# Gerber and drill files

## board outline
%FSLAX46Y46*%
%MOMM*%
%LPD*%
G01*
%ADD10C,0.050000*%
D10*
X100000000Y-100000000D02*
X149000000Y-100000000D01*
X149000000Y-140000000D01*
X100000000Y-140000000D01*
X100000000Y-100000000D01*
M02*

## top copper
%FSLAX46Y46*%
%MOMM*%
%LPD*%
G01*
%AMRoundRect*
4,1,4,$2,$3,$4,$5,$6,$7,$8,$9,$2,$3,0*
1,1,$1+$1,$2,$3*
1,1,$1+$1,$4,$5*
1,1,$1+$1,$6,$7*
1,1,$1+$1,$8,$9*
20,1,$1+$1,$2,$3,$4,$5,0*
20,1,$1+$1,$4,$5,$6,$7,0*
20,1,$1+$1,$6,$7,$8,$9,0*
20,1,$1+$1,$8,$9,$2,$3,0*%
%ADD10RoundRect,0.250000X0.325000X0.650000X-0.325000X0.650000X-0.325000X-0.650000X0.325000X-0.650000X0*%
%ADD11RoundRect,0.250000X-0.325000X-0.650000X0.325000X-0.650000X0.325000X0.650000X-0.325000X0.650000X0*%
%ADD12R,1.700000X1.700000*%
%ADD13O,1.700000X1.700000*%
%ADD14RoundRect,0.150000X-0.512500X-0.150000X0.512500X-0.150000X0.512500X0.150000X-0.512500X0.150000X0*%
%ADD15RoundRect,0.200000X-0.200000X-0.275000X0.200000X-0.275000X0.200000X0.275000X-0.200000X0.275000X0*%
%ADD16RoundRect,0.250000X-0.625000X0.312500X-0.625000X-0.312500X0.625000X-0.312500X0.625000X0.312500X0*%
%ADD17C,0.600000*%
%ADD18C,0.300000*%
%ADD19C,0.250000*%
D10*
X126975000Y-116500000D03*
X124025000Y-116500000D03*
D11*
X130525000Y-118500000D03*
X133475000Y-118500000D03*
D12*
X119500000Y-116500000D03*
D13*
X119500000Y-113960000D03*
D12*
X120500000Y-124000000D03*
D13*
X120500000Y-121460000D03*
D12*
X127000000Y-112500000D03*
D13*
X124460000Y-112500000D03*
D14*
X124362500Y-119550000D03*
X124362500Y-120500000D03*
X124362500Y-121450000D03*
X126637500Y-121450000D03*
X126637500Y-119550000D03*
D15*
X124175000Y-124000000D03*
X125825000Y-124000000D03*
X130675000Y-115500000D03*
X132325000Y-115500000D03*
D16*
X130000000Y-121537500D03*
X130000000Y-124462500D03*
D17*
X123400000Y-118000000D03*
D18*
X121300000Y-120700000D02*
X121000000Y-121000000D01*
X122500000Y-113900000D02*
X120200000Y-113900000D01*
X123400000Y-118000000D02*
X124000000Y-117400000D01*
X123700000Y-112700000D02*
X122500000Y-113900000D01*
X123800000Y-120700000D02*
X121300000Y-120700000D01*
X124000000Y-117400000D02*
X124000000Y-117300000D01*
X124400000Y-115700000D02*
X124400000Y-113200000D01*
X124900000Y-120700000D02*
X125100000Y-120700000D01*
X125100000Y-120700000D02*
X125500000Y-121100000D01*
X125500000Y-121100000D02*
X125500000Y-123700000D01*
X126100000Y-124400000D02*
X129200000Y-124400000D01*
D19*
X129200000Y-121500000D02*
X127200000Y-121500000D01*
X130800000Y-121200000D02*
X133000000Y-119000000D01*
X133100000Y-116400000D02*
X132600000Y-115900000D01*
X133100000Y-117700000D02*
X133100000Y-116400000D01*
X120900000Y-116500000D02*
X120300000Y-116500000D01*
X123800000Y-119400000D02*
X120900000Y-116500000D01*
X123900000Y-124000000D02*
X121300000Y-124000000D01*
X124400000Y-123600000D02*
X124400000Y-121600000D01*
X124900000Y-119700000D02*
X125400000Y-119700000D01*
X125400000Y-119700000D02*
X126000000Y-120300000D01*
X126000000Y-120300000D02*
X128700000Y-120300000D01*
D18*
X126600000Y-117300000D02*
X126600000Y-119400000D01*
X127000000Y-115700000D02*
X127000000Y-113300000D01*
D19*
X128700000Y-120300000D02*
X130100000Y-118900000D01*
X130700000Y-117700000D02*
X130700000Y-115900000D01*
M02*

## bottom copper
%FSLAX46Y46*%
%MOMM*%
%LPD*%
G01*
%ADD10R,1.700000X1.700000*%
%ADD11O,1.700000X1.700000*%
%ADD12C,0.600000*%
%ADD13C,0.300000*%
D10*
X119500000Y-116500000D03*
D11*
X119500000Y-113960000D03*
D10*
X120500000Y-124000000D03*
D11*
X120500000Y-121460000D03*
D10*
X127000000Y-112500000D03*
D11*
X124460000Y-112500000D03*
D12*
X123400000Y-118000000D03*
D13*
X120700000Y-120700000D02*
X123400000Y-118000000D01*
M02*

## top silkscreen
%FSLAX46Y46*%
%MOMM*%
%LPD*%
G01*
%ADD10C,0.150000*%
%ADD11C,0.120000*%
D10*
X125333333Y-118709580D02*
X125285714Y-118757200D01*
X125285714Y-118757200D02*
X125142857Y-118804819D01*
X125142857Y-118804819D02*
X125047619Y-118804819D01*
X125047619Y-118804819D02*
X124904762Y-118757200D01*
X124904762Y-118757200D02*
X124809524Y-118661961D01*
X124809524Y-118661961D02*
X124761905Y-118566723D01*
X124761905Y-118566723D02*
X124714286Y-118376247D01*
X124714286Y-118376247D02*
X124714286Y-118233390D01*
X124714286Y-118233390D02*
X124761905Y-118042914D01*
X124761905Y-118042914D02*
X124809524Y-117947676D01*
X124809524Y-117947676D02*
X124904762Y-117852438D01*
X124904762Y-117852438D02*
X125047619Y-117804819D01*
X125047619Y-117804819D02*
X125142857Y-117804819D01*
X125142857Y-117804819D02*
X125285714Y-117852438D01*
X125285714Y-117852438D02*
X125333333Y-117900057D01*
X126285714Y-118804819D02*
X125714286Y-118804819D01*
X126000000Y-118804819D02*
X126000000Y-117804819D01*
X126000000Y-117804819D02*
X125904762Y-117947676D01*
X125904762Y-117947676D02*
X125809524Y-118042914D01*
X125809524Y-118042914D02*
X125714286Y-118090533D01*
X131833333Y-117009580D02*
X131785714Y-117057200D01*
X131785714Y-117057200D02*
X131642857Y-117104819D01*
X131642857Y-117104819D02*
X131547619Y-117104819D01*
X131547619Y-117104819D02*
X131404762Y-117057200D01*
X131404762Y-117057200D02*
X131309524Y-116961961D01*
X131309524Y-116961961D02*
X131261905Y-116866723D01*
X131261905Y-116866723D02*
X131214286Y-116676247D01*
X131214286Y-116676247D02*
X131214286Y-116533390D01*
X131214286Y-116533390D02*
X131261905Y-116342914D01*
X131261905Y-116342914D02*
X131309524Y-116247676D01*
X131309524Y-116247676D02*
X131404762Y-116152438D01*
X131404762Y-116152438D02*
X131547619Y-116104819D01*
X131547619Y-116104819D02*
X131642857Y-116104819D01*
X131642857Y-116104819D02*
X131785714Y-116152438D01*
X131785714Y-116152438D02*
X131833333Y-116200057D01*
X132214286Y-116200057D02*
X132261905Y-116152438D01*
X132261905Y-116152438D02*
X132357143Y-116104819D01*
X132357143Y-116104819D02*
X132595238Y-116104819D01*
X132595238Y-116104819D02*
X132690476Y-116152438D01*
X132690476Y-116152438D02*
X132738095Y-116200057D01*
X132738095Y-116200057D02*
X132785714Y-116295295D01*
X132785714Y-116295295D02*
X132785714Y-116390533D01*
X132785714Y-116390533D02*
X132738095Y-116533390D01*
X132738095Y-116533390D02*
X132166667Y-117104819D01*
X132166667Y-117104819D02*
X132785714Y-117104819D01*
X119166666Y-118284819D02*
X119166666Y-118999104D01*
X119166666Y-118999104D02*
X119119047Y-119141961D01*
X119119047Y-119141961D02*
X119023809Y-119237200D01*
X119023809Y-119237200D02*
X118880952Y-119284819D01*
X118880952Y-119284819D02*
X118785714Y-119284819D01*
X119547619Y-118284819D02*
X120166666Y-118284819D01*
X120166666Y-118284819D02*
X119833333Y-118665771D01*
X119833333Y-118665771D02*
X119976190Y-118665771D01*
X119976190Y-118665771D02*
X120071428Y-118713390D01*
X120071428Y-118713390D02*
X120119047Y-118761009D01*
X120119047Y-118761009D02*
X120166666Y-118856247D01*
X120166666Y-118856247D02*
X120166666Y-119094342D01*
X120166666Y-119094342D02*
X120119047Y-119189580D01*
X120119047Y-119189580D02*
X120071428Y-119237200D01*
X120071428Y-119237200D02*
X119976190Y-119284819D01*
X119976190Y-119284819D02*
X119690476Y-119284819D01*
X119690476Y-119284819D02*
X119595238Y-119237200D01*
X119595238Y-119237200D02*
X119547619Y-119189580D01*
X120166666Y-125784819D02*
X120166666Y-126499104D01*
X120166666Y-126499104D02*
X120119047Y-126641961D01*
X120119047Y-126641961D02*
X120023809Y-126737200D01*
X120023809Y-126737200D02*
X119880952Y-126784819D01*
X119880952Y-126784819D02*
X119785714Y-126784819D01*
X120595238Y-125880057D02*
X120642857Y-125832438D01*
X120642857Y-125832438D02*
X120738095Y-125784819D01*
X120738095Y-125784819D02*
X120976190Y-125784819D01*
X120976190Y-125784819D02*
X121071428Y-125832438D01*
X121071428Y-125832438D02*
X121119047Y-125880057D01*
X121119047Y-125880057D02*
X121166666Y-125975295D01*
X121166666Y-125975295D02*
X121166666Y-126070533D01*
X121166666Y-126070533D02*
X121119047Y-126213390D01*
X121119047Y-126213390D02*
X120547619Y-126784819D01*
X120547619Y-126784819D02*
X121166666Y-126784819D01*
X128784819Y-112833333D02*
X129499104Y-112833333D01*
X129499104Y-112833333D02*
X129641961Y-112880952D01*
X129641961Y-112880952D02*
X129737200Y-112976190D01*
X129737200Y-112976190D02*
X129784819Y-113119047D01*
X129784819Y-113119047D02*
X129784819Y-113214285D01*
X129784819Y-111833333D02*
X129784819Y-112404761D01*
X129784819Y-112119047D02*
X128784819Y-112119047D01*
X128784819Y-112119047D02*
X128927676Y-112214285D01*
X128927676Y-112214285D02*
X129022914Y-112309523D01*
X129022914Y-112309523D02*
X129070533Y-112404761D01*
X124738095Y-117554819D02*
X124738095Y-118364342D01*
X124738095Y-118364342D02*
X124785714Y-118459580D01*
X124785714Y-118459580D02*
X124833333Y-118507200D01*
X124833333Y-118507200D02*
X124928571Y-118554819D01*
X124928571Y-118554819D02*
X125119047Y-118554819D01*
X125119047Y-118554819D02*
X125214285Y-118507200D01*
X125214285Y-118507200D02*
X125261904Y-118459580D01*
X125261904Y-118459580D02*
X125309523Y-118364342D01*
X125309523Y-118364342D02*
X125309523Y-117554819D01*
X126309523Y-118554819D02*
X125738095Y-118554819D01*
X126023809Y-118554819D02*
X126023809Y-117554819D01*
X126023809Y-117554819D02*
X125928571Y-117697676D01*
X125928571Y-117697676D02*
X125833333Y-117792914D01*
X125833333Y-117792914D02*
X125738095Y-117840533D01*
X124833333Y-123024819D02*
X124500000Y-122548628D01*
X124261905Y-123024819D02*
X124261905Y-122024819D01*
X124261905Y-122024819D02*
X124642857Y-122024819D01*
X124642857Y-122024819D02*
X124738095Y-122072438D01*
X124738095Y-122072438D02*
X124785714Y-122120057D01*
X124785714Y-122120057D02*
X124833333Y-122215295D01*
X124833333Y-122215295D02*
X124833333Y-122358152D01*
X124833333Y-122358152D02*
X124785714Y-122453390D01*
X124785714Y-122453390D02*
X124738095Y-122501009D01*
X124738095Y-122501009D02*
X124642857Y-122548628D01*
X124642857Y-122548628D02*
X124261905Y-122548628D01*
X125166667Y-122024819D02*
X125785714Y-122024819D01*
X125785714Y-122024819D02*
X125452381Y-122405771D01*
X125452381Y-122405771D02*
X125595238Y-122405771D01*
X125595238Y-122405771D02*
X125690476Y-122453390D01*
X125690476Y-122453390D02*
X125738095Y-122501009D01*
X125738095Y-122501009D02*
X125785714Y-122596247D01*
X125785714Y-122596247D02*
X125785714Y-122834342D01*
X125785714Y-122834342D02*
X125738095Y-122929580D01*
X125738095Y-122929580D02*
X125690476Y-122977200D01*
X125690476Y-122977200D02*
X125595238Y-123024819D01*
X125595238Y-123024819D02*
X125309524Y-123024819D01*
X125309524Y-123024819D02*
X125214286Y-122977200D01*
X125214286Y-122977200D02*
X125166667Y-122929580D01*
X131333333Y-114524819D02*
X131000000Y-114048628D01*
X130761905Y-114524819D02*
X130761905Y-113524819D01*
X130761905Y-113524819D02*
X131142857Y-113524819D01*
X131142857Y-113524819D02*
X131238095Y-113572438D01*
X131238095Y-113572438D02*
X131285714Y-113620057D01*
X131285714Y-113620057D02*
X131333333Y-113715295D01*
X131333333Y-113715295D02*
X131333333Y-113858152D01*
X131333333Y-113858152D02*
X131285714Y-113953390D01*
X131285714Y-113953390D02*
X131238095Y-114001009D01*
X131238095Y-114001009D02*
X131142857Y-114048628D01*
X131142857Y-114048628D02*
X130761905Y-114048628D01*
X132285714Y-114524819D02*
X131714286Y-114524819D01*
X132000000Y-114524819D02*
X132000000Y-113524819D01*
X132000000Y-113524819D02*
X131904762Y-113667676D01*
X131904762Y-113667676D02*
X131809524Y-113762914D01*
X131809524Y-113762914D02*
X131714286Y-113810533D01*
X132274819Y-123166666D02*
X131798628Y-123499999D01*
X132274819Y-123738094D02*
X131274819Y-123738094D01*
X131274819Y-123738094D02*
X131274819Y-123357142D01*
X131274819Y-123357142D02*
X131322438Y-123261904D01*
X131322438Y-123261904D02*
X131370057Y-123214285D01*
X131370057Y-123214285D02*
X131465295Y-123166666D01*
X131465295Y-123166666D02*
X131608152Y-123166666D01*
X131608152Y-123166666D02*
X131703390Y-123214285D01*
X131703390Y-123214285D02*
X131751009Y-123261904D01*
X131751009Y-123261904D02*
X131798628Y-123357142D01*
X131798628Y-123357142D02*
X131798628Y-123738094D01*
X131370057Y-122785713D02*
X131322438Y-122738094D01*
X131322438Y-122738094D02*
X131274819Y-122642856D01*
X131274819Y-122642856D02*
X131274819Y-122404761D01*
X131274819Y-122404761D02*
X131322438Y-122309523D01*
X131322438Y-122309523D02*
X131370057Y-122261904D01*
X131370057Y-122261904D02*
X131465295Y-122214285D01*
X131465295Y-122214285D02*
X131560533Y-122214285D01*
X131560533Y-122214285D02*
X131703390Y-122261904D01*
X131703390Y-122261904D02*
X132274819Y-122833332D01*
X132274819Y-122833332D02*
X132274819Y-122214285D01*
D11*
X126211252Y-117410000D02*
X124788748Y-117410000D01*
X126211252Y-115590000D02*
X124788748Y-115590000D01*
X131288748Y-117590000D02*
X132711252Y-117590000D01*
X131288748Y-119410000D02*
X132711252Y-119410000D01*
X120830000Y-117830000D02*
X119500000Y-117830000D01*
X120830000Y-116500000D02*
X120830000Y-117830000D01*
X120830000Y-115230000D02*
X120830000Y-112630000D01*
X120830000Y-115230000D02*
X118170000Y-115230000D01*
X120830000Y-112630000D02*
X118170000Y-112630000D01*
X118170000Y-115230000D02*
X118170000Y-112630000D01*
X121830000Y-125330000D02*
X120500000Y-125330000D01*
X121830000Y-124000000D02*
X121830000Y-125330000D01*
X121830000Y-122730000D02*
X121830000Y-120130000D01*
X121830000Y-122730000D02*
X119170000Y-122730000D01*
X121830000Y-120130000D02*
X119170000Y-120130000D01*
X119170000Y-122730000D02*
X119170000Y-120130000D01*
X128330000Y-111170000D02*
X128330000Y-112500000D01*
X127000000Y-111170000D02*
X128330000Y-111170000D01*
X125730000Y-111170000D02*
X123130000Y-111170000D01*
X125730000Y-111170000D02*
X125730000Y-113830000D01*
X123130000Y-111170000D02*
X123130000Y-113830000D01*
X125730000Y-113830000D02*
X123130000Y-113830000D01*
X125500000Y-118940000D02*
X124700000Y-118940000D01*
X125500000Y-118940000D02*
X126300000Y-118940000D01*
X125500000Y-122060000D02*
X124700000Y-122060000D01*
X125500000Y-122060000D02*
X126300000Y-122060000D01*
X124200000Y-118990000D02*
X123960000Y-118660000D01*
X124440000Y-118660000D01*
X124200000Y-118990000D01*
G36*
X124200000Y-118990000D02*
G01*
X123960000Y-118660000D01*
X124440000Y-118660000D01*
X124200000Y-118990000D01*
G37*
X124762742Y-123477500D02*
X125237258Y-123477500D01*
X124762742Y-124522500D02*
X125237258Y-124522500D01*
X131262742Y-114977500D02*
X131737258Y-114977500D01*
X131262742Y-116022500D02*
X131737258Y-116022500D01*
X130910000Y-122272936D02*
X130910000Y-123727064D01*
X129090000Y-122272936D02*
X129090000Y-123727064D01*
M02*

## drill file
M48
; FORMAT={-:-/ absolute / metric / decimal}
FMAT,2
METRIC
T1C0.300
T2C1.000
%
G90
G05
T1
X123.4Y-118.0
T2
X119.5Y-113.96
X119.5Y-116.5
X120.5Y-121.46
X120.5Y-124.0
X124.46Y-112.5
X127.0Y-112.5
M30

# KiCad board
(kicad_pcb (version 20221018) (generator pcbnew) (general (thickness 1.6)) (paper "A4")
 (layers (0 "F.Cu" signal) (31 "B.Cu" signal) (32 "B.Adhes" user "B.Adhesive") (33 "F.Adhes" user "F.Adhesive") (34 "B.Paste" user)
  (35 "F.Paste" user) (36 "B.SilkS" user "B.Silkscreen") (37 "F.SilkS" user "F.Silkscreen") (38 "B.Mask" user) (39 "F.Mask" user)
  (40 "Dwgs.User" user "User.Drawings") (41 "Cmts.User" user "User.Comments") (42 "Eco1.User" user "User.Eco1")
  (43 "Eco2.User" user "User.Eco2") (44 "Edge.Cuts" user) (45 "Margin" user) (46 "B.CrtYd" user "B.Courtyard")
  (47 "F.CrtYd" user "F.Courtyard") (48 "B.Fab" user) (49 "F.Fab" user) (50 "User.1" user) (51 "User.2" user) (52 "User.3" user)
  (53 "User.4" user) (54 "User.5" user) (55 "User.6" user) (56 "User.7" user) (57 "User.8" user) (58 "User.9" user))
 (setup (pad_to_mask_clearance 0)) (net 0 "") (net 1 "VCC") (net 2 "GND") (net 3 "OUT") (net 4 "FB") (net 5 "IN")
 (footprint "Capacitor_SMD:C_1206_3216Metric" (layer "F.Cu") (at 125.5 116.5 180)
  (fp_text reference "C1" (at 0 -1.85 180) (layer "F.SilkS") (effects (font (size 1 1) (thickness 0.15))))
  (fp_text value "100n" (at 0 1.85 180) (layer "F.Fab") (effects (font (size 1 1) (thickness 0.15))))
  (fp_line (start -0.711252 -0.91) (end 0.711252 -0.91) (stroke (width 0.12) (type solid)) (layer "F.SilkS"))
  (fp_line (start -0.711252 0.91) (end 0.711252 0.91) (stroke (width 0.12) (type solid)) (layer "F.SilkS"))
  (pad "1" smd roundrect (at -1.475 0 180) (size 1.15 1.8) (layers "F.Cu" "F.Paste" "F.Mask") (roundrect_rratio 0.217391) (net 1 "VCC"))
  (pad "2" smd roundrect (at 1.475 0 180) (size 1.15 1.8) (layers "F.Cu" "F.Paste" "F.Mask") (roundrect_rratio 0.217391) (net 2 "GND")))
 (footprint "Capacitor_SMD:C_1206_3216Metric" (layer "F.Cu") (at 132 118.5)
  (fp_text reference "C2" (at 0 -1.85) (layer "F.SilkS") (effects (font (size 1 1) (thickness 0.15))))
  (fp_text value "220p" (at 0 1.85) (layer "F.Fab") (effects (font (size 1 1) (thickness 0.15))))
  (fp_line (start -0.711252 -0.91) (end 0.711252 -0.91) (stroke (width 0.12) (type solid)) (layer "F.SilkS"))
  (fp_line (start -0.711252 0.91) (end 0.711252 0.91) (stroke (width 0.12) (type solid)) (layer "F.SilkS"))
  (pad "1" smd roundrect (at -1.475 0) (size 1.15 1.8) (layers "F.Cu" "F.Paste" "F.Mask") (roundrect_rratio 0.217391) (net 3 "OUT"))
  (pad "2" smd roundrect (at 1.475 0) (size 1.15 1.8) (layers "F.Cu" "F.Paste" "F.Mask") (roundrect_rratio 0.217391) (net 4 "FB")))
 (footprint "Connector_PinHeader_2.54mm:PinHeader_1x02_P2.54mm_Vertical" (layer "F.Cu") (at 119.5 116.5 180)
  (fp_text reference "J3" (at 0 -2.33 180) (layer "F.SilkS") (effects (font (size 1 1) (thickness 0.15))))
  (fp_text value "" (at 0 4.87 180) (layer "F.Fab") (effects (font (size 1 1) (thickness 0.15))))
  (fp_line (start -1.33 -1.33) (end 0 -1.33) (stroke (width 0.12) (type solid)) (layer "F.SilkS"))
  (fp_line (start -1.33 0) (end -1.33 -1.33) (stroke (width 0.12) (type solid)) (layer "F.SilkS"))
  (fp_line (start -1.33 1.27) (end -1.33 3.87) (stroke (width 0.12) (type solid)) (layer "F.SilkS"))
  (fp_line (start -1.33 1.27) (end 1.33 1.27) (stroke (width 0.12) (type solid)) (layer "F.SilkS"))
  (fp_line (start -1.33 3.87) (end 1.33 3.87) (stroke (width 0.12) (type solid)) (layer "F.SilkS"))
  (fp_line (start 1.33 1.27) (end 1.33 3.87) (stroke (width 0.12) (type solid)) (layer "F.SilkS"))
  (pad "1" thru_hole rect (at 0 0 180) (size 1.7 1.7) (drill 1) (layers "*.Cu" "*.Mask") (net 3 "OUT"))
  (pad "2" thru_hole oval (at 0 2.54 180) (size 1.7 1.7) (drill 1) (layers "*.Cu" "*.Mask") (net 2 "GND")))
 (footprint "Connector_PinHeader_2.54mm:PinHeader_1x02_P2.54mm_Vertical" (layer "F.Cu") (at 120.5 124 180)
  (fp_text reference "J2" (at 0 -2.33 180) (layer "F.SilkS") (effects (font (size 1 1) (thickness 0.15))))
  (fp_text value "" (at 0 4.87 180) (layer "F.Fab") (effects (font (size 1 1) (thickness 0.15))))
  (fp_line (start -1.33 -1.33) (end 0 -1.33) (stroke (width 0.12) (type solid)) (layer "F.SilkS"))
  (fp_line (start -1.33 0) (end -1.33 -1.33) (stroke (width 0.12) (type solid)) (layer "F.SilkS"))
  (fp_line (start -1.33 1.27) (end -1.33 3.87) (stroke (width 0.12) (type solid)) (layer "F.SilkS"))
  (fp_line (start -1.33 1.27) (end 1.33 1.27) (stroke (width 0.12) (type solid)) (layer "F.SilkS"))
  (fp_line (start -1.33 3.87) (end 1.33 3.87) (stroke (width 0.12) (type solid)) (layer "F.SilkS"))
  (fp_line (start 1.33 1.27) (end 1.33 3.87) (stroke (width 0.12) (type solid)) (layer "F.SilkS"))
  (pad "1" thru_hole rect (at 0 0 180) (size 1.7 1.7) (drill 1) (layers "*.Cu" "*.Mask") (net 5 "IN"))
  (pad "2" thru_hole oval (at 0 2.54 180) (size 1.7 1.7) (drill 1) (layers "*.Cu" "*.Mask") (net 2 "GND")))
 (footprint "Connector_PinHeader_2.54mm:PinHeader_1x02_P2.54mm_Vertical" (layer "F.Cu") (at 127 112.5 -90)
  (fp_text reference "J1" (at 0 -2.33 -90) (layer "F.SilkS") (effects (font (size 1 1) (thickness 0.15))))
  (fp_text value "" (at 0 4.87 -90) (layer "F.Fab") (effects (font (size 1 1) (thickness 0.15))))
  (fp_line (start -1.33 -1.33) (end 0 -1.33) (stroke (width 0.12) (type solid)) (layer "F.SilkS"))
  (fp_line (start -1.33 0) (end -1.33 -1.33) (stroke (width 0.12) (type solid)) (layer "F.SilkS"))
  (fp_line (start -1.33 1.27) (end -1.33 3.87) (stroke (width 0.12) (type solid)) (layer "F.SilkS"))
  (fp_line (start -1.33 1.27) (end 1.33 1.27) (stroke (width 0.12) (type solid)) (layer "F.SilkS"))
  (fp_line (start -1.33 3.87) (end 1.33 3.87) (stroke (width 0.12) (type solid)) (layer "F.SilkS"))
  (fp_line (start 1.33 1.27) (end 1.33 3.87) (stroke (width 0.12) (type solid)) (layer "F.SilkS"))
  (pad "1" thru_hole rect (at 0 0 270) (size 1.7 1.7) (drill 1) (layers "*.Cu" "*.Mask") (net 1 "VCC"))
  (pad "2" thru_hole oval (at 0 2.54 270) (size 1.7 1.7) (drill 1) (layers "*.Cu" "*.Mask") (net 2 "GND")))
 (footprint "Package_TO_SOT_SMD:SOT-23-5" (layer "F.Cu") (at 125.5 120.5)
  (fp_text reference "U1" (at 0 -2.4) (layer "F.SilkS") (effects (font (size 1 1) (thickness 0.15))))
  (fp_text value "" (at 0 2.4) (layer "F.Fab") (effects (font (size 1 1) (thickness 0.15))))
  (fp_line (start 0 -1.56) (end -0.8 -1.56) (stroke (width 0.12) (type solid)) (layer "F.SilkS"))
  (fp_line (start 0 -1.56) (end 0.8 -1.56) (stroke (width 0.12) (type solid)) (layer "F.SilkS"))
  (fp_line (start 0 1.56) (end -0.8 1.56) (stroke (width 0.12) (type solid)) (layer "F.SilkS"))
  (fp_line (start 0 1.56) (end 0.8 1.56) (stroke (width 0.12) (type solid)) (layer "F.SilkS"))
  (fp_poly
   (pts (xy -1.3 -1.51) (xy -1.54 -1.84) (xy -1.06 -1.84) (xy -1.3 -1.51)) (stroke (width 0.12) (type solid)) (fill solid) (layer "F.SilkS"))
  (pad "1" smd roundrect (at -1.1375 -0.95) (size 1.325 0.6) (layers "F.Cu" "F.Paste" "F.Mask") (roundrect_rratio 0.25) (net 3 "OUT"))
  (pad "2" smd roundrect (at -1.1375 0) (size 1.325 0.6) (layers "F.Cu" "F.Paste" "F.Mask") (roundrect_rratio 0.25) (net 2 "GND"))
  (pad "3" smd roundrect (at -1.1375 0.95) (size 1.325 0.6) (layers "F.Cu" "F.Paste" "F.Mask") (roundrect_rratio 0.25) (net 5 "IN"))
  (pad "4" smd roundrect (at 1.1375 0.95) (size 1.325 0.6) (layers "F.Cu" "F.Paste" "F.Mask") (roundrect_rratio 0.25) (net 4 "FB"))
  (pad "5" smd roundrect (at 1.1375 -0.95) (size 1.325 0.6) (layers "F.Cu" "F.Paste" "F.Mask") (roundrect_rratio 0.25) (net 1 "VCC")))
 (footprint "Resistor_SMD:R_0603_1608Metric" (layer "F.Cu") (at 125 124)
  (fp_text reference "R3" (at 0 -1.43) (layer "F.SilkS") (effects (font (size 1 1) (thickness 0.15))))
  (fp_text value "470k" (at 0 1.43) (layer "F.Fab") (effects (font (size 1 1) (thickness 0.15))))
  (fp_line (start -0.237258 -0.5225) (end 0.237258 -0.5225) (stroke (width 0.12) (type solid)) (layer "F.SilkS"))
  (fp_line (start -0.237258 0.5225) (end 0.237258 0.5225) (stroke (width 0.12) (type solid)) (layer "F.SilkS"))
  (pad "1" smd roundrect (at -0.825 0) (size 0.8 0.95) (layers "F.Cu" "F.Paste" "F.Mask") (roundrect_rratio 0.25) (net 5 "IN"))
  (pad "2" smd roundrect (at 0.825 0) (size 0.8 0.95) (layers "F.Cu" "F.Paste" "F.Mask") (roundrect_rratio 0.25) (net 2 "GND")))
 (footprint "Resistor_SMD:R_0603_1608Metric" (layer "F.Cu") (at 131.5 115.5)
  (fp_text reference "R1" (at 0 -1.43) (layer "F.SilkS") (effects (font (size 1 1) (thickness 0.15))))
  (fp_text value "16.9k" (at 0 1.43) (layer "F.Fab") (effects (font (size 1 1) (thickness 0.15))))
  (fp_line (start -0.237258 -0.5225) (end 0.237258 -0.5225) (stroke (width 0.12) (type solid)) (layer "F.SilkS"))
  (fp_line (start -0.237258 0.5225) (end 0.237258 0.5225) (stroke (width 0.12) (type solid)) (layer "F.SilkS"))
  (pad "1" smd roundrect (at -0.825 0) (size 0.8 0.95) (layers "F.Cu" "F.Paste" "F.Mask") (roundrect_rratio 0.25) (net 3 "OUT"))
  (pad "2" smd roundrect (at 0.825 0) (size 0.8 0.95) (layers "F.Cu" "F.Paste" "F.Mask") (roundrect_rratio 0.25) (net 4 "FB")))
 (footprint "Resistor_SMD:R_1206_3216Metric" (layer "F.Cu") (at 130 123 -90)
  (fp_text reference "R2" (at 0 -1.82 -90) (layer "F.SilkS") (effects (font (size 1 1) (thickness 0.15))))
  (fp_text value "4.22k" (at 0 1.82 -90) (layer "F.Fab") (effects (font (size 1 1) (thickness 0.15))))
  (fp_line (start -0.727064 -0.91) (end 0.727064 -0.91) (stroke (width 0.12) (type solid)) (layer "F.SilkS"))
  (fp_line (start -0.727064 0.91) (end 0.727064 0.91) (stroke (width 0.12) (type solid)) (layer "F.SilkS"))
  (pad "1" smd roundrect (at -1.4625 0 270) (size 1.125 1.75) (layers "F.Cu" "F.Paste" "F.Mask") (roundrect_rratio 0.222222) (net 4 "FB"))
  (pad "2" smd roundrect (at 1.4625 0 270) (size 1.125 1.75) (layers "F.Cu" "F.Paste" "F.Mask") (roundrect_rratio 0.222222) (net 2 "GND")))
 (gr_rect (start 100 100) (end 149 140) (stroke (width 0.05) (type default)) (fill none) (layer "Edge.Cuts"))
 (segment (start 121.3 120.7) (end 121 121) (width 0.3) (layer "F.Cu") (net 2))
 (segment (start 122.5 113.9) (end 120.2 113.9) (width 0.3) (layer "F.Cu") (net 2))
 (segment (start 123.4 118) (end 124 117.4) (width 0.3) (layer "F.Cu") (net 2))
 (segment (start 123.7 112.7) (end 122.5 113.9) (width 0.3) (layer "F.Cu") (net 2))
 (segment (start 123.8 120.7) (end 121.3 120.7) (width 0.3) (layer "F.Cu") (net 2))
 (segment (start 124 117.4) (end 124 117.3) (width 0.3) (layer "F.Cu") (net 2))
 (segment (start 124.4 115.7) (end 124.4 113.2) (width 0.3) (layer "F.Cu") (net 2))
 (segment (start 124.9 120.7) (end 125.1 120.7) (width 0.3) (layer "F.Cu") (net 2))
 (segment (start 125.1 120.7) (end 125.5 121.1) (width 0.3) (layer "F.Cu") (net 2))
 (segment (start 125.5 121.1) (end 125.5 123.7) (width 0.3) (layer "F.Cu") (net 2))
 (segment (start 126.1 124.4) (end 129.2 124.4) (width 0.3) (layer "F.Cu") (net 2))
 (segment (start 129.2 121.5) (end 127.2 121.5) (width 0.25) (layer "F.Cu") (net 4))
 (segment (start 130.8 121.2) (end 133 119) (width 0.25) (layer "F.Cu") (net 4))
 (segment (start 133.1 116.4) (end 132.6 115.9) (width 0.25) (layer "F.Cu") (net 4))
 (segment (start 133.1 117.7) (end 133.1 116.4) (width 0.25) (layer "F.Cu") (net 4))
 (via (at 123.4 118) (size 0.6) (drill 0.3) (layers "F.Cu" "B.Cu") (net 2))
 (segment (start 120.7 120.7) (end 123.4 118) (width 0.3) (layer "B.Cu") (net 2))
 (segment (start 120.9 116.5) (end 120.3 116.5) (width 0.25) (layer "F.Cu") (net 3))
 (segment (start 123.8 119.4) (end 120.9 116.5) (width 0.25) (layer "F.Cu") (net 3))
 (segment (start 123.9 124) (end 121.3 124) (width 0.25) (layer "F.Cu") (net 5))
 (segment (start 124.4 123.6) (end 124.4 121.6) (width 0.25) (layer "F.Cu") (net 5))
 (segment (start 124.9 119.7) (end 125.4 119.7) (width 0.25) (layer "F.Cu") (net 3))
 (segment (start 125.4 119.7) (end 126 120.3) (width 0.25) (layer "F.Cu") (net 3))
 (segment (start 126 120.3) (end 128.7 120.3) (width 0.25) (layer "F.Cu") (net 3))
 (segment (start 126.6 117.3) (end 126.6 119.4) (width 0.3) (layer "F.Cu") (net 1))
 (segment (start 127 115.7) (end 127 113.3) (width 0.3) (layer "F.Cu") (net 1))
 (segment (start 128.7 120.3) (end 130.1 118.9) (width 0.25) (layer "F.Cu") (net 3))
 (segment (start 130.7 117.7) (end 130.7 115.9) (width 0.25) (layer "F.Cu") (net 3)))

